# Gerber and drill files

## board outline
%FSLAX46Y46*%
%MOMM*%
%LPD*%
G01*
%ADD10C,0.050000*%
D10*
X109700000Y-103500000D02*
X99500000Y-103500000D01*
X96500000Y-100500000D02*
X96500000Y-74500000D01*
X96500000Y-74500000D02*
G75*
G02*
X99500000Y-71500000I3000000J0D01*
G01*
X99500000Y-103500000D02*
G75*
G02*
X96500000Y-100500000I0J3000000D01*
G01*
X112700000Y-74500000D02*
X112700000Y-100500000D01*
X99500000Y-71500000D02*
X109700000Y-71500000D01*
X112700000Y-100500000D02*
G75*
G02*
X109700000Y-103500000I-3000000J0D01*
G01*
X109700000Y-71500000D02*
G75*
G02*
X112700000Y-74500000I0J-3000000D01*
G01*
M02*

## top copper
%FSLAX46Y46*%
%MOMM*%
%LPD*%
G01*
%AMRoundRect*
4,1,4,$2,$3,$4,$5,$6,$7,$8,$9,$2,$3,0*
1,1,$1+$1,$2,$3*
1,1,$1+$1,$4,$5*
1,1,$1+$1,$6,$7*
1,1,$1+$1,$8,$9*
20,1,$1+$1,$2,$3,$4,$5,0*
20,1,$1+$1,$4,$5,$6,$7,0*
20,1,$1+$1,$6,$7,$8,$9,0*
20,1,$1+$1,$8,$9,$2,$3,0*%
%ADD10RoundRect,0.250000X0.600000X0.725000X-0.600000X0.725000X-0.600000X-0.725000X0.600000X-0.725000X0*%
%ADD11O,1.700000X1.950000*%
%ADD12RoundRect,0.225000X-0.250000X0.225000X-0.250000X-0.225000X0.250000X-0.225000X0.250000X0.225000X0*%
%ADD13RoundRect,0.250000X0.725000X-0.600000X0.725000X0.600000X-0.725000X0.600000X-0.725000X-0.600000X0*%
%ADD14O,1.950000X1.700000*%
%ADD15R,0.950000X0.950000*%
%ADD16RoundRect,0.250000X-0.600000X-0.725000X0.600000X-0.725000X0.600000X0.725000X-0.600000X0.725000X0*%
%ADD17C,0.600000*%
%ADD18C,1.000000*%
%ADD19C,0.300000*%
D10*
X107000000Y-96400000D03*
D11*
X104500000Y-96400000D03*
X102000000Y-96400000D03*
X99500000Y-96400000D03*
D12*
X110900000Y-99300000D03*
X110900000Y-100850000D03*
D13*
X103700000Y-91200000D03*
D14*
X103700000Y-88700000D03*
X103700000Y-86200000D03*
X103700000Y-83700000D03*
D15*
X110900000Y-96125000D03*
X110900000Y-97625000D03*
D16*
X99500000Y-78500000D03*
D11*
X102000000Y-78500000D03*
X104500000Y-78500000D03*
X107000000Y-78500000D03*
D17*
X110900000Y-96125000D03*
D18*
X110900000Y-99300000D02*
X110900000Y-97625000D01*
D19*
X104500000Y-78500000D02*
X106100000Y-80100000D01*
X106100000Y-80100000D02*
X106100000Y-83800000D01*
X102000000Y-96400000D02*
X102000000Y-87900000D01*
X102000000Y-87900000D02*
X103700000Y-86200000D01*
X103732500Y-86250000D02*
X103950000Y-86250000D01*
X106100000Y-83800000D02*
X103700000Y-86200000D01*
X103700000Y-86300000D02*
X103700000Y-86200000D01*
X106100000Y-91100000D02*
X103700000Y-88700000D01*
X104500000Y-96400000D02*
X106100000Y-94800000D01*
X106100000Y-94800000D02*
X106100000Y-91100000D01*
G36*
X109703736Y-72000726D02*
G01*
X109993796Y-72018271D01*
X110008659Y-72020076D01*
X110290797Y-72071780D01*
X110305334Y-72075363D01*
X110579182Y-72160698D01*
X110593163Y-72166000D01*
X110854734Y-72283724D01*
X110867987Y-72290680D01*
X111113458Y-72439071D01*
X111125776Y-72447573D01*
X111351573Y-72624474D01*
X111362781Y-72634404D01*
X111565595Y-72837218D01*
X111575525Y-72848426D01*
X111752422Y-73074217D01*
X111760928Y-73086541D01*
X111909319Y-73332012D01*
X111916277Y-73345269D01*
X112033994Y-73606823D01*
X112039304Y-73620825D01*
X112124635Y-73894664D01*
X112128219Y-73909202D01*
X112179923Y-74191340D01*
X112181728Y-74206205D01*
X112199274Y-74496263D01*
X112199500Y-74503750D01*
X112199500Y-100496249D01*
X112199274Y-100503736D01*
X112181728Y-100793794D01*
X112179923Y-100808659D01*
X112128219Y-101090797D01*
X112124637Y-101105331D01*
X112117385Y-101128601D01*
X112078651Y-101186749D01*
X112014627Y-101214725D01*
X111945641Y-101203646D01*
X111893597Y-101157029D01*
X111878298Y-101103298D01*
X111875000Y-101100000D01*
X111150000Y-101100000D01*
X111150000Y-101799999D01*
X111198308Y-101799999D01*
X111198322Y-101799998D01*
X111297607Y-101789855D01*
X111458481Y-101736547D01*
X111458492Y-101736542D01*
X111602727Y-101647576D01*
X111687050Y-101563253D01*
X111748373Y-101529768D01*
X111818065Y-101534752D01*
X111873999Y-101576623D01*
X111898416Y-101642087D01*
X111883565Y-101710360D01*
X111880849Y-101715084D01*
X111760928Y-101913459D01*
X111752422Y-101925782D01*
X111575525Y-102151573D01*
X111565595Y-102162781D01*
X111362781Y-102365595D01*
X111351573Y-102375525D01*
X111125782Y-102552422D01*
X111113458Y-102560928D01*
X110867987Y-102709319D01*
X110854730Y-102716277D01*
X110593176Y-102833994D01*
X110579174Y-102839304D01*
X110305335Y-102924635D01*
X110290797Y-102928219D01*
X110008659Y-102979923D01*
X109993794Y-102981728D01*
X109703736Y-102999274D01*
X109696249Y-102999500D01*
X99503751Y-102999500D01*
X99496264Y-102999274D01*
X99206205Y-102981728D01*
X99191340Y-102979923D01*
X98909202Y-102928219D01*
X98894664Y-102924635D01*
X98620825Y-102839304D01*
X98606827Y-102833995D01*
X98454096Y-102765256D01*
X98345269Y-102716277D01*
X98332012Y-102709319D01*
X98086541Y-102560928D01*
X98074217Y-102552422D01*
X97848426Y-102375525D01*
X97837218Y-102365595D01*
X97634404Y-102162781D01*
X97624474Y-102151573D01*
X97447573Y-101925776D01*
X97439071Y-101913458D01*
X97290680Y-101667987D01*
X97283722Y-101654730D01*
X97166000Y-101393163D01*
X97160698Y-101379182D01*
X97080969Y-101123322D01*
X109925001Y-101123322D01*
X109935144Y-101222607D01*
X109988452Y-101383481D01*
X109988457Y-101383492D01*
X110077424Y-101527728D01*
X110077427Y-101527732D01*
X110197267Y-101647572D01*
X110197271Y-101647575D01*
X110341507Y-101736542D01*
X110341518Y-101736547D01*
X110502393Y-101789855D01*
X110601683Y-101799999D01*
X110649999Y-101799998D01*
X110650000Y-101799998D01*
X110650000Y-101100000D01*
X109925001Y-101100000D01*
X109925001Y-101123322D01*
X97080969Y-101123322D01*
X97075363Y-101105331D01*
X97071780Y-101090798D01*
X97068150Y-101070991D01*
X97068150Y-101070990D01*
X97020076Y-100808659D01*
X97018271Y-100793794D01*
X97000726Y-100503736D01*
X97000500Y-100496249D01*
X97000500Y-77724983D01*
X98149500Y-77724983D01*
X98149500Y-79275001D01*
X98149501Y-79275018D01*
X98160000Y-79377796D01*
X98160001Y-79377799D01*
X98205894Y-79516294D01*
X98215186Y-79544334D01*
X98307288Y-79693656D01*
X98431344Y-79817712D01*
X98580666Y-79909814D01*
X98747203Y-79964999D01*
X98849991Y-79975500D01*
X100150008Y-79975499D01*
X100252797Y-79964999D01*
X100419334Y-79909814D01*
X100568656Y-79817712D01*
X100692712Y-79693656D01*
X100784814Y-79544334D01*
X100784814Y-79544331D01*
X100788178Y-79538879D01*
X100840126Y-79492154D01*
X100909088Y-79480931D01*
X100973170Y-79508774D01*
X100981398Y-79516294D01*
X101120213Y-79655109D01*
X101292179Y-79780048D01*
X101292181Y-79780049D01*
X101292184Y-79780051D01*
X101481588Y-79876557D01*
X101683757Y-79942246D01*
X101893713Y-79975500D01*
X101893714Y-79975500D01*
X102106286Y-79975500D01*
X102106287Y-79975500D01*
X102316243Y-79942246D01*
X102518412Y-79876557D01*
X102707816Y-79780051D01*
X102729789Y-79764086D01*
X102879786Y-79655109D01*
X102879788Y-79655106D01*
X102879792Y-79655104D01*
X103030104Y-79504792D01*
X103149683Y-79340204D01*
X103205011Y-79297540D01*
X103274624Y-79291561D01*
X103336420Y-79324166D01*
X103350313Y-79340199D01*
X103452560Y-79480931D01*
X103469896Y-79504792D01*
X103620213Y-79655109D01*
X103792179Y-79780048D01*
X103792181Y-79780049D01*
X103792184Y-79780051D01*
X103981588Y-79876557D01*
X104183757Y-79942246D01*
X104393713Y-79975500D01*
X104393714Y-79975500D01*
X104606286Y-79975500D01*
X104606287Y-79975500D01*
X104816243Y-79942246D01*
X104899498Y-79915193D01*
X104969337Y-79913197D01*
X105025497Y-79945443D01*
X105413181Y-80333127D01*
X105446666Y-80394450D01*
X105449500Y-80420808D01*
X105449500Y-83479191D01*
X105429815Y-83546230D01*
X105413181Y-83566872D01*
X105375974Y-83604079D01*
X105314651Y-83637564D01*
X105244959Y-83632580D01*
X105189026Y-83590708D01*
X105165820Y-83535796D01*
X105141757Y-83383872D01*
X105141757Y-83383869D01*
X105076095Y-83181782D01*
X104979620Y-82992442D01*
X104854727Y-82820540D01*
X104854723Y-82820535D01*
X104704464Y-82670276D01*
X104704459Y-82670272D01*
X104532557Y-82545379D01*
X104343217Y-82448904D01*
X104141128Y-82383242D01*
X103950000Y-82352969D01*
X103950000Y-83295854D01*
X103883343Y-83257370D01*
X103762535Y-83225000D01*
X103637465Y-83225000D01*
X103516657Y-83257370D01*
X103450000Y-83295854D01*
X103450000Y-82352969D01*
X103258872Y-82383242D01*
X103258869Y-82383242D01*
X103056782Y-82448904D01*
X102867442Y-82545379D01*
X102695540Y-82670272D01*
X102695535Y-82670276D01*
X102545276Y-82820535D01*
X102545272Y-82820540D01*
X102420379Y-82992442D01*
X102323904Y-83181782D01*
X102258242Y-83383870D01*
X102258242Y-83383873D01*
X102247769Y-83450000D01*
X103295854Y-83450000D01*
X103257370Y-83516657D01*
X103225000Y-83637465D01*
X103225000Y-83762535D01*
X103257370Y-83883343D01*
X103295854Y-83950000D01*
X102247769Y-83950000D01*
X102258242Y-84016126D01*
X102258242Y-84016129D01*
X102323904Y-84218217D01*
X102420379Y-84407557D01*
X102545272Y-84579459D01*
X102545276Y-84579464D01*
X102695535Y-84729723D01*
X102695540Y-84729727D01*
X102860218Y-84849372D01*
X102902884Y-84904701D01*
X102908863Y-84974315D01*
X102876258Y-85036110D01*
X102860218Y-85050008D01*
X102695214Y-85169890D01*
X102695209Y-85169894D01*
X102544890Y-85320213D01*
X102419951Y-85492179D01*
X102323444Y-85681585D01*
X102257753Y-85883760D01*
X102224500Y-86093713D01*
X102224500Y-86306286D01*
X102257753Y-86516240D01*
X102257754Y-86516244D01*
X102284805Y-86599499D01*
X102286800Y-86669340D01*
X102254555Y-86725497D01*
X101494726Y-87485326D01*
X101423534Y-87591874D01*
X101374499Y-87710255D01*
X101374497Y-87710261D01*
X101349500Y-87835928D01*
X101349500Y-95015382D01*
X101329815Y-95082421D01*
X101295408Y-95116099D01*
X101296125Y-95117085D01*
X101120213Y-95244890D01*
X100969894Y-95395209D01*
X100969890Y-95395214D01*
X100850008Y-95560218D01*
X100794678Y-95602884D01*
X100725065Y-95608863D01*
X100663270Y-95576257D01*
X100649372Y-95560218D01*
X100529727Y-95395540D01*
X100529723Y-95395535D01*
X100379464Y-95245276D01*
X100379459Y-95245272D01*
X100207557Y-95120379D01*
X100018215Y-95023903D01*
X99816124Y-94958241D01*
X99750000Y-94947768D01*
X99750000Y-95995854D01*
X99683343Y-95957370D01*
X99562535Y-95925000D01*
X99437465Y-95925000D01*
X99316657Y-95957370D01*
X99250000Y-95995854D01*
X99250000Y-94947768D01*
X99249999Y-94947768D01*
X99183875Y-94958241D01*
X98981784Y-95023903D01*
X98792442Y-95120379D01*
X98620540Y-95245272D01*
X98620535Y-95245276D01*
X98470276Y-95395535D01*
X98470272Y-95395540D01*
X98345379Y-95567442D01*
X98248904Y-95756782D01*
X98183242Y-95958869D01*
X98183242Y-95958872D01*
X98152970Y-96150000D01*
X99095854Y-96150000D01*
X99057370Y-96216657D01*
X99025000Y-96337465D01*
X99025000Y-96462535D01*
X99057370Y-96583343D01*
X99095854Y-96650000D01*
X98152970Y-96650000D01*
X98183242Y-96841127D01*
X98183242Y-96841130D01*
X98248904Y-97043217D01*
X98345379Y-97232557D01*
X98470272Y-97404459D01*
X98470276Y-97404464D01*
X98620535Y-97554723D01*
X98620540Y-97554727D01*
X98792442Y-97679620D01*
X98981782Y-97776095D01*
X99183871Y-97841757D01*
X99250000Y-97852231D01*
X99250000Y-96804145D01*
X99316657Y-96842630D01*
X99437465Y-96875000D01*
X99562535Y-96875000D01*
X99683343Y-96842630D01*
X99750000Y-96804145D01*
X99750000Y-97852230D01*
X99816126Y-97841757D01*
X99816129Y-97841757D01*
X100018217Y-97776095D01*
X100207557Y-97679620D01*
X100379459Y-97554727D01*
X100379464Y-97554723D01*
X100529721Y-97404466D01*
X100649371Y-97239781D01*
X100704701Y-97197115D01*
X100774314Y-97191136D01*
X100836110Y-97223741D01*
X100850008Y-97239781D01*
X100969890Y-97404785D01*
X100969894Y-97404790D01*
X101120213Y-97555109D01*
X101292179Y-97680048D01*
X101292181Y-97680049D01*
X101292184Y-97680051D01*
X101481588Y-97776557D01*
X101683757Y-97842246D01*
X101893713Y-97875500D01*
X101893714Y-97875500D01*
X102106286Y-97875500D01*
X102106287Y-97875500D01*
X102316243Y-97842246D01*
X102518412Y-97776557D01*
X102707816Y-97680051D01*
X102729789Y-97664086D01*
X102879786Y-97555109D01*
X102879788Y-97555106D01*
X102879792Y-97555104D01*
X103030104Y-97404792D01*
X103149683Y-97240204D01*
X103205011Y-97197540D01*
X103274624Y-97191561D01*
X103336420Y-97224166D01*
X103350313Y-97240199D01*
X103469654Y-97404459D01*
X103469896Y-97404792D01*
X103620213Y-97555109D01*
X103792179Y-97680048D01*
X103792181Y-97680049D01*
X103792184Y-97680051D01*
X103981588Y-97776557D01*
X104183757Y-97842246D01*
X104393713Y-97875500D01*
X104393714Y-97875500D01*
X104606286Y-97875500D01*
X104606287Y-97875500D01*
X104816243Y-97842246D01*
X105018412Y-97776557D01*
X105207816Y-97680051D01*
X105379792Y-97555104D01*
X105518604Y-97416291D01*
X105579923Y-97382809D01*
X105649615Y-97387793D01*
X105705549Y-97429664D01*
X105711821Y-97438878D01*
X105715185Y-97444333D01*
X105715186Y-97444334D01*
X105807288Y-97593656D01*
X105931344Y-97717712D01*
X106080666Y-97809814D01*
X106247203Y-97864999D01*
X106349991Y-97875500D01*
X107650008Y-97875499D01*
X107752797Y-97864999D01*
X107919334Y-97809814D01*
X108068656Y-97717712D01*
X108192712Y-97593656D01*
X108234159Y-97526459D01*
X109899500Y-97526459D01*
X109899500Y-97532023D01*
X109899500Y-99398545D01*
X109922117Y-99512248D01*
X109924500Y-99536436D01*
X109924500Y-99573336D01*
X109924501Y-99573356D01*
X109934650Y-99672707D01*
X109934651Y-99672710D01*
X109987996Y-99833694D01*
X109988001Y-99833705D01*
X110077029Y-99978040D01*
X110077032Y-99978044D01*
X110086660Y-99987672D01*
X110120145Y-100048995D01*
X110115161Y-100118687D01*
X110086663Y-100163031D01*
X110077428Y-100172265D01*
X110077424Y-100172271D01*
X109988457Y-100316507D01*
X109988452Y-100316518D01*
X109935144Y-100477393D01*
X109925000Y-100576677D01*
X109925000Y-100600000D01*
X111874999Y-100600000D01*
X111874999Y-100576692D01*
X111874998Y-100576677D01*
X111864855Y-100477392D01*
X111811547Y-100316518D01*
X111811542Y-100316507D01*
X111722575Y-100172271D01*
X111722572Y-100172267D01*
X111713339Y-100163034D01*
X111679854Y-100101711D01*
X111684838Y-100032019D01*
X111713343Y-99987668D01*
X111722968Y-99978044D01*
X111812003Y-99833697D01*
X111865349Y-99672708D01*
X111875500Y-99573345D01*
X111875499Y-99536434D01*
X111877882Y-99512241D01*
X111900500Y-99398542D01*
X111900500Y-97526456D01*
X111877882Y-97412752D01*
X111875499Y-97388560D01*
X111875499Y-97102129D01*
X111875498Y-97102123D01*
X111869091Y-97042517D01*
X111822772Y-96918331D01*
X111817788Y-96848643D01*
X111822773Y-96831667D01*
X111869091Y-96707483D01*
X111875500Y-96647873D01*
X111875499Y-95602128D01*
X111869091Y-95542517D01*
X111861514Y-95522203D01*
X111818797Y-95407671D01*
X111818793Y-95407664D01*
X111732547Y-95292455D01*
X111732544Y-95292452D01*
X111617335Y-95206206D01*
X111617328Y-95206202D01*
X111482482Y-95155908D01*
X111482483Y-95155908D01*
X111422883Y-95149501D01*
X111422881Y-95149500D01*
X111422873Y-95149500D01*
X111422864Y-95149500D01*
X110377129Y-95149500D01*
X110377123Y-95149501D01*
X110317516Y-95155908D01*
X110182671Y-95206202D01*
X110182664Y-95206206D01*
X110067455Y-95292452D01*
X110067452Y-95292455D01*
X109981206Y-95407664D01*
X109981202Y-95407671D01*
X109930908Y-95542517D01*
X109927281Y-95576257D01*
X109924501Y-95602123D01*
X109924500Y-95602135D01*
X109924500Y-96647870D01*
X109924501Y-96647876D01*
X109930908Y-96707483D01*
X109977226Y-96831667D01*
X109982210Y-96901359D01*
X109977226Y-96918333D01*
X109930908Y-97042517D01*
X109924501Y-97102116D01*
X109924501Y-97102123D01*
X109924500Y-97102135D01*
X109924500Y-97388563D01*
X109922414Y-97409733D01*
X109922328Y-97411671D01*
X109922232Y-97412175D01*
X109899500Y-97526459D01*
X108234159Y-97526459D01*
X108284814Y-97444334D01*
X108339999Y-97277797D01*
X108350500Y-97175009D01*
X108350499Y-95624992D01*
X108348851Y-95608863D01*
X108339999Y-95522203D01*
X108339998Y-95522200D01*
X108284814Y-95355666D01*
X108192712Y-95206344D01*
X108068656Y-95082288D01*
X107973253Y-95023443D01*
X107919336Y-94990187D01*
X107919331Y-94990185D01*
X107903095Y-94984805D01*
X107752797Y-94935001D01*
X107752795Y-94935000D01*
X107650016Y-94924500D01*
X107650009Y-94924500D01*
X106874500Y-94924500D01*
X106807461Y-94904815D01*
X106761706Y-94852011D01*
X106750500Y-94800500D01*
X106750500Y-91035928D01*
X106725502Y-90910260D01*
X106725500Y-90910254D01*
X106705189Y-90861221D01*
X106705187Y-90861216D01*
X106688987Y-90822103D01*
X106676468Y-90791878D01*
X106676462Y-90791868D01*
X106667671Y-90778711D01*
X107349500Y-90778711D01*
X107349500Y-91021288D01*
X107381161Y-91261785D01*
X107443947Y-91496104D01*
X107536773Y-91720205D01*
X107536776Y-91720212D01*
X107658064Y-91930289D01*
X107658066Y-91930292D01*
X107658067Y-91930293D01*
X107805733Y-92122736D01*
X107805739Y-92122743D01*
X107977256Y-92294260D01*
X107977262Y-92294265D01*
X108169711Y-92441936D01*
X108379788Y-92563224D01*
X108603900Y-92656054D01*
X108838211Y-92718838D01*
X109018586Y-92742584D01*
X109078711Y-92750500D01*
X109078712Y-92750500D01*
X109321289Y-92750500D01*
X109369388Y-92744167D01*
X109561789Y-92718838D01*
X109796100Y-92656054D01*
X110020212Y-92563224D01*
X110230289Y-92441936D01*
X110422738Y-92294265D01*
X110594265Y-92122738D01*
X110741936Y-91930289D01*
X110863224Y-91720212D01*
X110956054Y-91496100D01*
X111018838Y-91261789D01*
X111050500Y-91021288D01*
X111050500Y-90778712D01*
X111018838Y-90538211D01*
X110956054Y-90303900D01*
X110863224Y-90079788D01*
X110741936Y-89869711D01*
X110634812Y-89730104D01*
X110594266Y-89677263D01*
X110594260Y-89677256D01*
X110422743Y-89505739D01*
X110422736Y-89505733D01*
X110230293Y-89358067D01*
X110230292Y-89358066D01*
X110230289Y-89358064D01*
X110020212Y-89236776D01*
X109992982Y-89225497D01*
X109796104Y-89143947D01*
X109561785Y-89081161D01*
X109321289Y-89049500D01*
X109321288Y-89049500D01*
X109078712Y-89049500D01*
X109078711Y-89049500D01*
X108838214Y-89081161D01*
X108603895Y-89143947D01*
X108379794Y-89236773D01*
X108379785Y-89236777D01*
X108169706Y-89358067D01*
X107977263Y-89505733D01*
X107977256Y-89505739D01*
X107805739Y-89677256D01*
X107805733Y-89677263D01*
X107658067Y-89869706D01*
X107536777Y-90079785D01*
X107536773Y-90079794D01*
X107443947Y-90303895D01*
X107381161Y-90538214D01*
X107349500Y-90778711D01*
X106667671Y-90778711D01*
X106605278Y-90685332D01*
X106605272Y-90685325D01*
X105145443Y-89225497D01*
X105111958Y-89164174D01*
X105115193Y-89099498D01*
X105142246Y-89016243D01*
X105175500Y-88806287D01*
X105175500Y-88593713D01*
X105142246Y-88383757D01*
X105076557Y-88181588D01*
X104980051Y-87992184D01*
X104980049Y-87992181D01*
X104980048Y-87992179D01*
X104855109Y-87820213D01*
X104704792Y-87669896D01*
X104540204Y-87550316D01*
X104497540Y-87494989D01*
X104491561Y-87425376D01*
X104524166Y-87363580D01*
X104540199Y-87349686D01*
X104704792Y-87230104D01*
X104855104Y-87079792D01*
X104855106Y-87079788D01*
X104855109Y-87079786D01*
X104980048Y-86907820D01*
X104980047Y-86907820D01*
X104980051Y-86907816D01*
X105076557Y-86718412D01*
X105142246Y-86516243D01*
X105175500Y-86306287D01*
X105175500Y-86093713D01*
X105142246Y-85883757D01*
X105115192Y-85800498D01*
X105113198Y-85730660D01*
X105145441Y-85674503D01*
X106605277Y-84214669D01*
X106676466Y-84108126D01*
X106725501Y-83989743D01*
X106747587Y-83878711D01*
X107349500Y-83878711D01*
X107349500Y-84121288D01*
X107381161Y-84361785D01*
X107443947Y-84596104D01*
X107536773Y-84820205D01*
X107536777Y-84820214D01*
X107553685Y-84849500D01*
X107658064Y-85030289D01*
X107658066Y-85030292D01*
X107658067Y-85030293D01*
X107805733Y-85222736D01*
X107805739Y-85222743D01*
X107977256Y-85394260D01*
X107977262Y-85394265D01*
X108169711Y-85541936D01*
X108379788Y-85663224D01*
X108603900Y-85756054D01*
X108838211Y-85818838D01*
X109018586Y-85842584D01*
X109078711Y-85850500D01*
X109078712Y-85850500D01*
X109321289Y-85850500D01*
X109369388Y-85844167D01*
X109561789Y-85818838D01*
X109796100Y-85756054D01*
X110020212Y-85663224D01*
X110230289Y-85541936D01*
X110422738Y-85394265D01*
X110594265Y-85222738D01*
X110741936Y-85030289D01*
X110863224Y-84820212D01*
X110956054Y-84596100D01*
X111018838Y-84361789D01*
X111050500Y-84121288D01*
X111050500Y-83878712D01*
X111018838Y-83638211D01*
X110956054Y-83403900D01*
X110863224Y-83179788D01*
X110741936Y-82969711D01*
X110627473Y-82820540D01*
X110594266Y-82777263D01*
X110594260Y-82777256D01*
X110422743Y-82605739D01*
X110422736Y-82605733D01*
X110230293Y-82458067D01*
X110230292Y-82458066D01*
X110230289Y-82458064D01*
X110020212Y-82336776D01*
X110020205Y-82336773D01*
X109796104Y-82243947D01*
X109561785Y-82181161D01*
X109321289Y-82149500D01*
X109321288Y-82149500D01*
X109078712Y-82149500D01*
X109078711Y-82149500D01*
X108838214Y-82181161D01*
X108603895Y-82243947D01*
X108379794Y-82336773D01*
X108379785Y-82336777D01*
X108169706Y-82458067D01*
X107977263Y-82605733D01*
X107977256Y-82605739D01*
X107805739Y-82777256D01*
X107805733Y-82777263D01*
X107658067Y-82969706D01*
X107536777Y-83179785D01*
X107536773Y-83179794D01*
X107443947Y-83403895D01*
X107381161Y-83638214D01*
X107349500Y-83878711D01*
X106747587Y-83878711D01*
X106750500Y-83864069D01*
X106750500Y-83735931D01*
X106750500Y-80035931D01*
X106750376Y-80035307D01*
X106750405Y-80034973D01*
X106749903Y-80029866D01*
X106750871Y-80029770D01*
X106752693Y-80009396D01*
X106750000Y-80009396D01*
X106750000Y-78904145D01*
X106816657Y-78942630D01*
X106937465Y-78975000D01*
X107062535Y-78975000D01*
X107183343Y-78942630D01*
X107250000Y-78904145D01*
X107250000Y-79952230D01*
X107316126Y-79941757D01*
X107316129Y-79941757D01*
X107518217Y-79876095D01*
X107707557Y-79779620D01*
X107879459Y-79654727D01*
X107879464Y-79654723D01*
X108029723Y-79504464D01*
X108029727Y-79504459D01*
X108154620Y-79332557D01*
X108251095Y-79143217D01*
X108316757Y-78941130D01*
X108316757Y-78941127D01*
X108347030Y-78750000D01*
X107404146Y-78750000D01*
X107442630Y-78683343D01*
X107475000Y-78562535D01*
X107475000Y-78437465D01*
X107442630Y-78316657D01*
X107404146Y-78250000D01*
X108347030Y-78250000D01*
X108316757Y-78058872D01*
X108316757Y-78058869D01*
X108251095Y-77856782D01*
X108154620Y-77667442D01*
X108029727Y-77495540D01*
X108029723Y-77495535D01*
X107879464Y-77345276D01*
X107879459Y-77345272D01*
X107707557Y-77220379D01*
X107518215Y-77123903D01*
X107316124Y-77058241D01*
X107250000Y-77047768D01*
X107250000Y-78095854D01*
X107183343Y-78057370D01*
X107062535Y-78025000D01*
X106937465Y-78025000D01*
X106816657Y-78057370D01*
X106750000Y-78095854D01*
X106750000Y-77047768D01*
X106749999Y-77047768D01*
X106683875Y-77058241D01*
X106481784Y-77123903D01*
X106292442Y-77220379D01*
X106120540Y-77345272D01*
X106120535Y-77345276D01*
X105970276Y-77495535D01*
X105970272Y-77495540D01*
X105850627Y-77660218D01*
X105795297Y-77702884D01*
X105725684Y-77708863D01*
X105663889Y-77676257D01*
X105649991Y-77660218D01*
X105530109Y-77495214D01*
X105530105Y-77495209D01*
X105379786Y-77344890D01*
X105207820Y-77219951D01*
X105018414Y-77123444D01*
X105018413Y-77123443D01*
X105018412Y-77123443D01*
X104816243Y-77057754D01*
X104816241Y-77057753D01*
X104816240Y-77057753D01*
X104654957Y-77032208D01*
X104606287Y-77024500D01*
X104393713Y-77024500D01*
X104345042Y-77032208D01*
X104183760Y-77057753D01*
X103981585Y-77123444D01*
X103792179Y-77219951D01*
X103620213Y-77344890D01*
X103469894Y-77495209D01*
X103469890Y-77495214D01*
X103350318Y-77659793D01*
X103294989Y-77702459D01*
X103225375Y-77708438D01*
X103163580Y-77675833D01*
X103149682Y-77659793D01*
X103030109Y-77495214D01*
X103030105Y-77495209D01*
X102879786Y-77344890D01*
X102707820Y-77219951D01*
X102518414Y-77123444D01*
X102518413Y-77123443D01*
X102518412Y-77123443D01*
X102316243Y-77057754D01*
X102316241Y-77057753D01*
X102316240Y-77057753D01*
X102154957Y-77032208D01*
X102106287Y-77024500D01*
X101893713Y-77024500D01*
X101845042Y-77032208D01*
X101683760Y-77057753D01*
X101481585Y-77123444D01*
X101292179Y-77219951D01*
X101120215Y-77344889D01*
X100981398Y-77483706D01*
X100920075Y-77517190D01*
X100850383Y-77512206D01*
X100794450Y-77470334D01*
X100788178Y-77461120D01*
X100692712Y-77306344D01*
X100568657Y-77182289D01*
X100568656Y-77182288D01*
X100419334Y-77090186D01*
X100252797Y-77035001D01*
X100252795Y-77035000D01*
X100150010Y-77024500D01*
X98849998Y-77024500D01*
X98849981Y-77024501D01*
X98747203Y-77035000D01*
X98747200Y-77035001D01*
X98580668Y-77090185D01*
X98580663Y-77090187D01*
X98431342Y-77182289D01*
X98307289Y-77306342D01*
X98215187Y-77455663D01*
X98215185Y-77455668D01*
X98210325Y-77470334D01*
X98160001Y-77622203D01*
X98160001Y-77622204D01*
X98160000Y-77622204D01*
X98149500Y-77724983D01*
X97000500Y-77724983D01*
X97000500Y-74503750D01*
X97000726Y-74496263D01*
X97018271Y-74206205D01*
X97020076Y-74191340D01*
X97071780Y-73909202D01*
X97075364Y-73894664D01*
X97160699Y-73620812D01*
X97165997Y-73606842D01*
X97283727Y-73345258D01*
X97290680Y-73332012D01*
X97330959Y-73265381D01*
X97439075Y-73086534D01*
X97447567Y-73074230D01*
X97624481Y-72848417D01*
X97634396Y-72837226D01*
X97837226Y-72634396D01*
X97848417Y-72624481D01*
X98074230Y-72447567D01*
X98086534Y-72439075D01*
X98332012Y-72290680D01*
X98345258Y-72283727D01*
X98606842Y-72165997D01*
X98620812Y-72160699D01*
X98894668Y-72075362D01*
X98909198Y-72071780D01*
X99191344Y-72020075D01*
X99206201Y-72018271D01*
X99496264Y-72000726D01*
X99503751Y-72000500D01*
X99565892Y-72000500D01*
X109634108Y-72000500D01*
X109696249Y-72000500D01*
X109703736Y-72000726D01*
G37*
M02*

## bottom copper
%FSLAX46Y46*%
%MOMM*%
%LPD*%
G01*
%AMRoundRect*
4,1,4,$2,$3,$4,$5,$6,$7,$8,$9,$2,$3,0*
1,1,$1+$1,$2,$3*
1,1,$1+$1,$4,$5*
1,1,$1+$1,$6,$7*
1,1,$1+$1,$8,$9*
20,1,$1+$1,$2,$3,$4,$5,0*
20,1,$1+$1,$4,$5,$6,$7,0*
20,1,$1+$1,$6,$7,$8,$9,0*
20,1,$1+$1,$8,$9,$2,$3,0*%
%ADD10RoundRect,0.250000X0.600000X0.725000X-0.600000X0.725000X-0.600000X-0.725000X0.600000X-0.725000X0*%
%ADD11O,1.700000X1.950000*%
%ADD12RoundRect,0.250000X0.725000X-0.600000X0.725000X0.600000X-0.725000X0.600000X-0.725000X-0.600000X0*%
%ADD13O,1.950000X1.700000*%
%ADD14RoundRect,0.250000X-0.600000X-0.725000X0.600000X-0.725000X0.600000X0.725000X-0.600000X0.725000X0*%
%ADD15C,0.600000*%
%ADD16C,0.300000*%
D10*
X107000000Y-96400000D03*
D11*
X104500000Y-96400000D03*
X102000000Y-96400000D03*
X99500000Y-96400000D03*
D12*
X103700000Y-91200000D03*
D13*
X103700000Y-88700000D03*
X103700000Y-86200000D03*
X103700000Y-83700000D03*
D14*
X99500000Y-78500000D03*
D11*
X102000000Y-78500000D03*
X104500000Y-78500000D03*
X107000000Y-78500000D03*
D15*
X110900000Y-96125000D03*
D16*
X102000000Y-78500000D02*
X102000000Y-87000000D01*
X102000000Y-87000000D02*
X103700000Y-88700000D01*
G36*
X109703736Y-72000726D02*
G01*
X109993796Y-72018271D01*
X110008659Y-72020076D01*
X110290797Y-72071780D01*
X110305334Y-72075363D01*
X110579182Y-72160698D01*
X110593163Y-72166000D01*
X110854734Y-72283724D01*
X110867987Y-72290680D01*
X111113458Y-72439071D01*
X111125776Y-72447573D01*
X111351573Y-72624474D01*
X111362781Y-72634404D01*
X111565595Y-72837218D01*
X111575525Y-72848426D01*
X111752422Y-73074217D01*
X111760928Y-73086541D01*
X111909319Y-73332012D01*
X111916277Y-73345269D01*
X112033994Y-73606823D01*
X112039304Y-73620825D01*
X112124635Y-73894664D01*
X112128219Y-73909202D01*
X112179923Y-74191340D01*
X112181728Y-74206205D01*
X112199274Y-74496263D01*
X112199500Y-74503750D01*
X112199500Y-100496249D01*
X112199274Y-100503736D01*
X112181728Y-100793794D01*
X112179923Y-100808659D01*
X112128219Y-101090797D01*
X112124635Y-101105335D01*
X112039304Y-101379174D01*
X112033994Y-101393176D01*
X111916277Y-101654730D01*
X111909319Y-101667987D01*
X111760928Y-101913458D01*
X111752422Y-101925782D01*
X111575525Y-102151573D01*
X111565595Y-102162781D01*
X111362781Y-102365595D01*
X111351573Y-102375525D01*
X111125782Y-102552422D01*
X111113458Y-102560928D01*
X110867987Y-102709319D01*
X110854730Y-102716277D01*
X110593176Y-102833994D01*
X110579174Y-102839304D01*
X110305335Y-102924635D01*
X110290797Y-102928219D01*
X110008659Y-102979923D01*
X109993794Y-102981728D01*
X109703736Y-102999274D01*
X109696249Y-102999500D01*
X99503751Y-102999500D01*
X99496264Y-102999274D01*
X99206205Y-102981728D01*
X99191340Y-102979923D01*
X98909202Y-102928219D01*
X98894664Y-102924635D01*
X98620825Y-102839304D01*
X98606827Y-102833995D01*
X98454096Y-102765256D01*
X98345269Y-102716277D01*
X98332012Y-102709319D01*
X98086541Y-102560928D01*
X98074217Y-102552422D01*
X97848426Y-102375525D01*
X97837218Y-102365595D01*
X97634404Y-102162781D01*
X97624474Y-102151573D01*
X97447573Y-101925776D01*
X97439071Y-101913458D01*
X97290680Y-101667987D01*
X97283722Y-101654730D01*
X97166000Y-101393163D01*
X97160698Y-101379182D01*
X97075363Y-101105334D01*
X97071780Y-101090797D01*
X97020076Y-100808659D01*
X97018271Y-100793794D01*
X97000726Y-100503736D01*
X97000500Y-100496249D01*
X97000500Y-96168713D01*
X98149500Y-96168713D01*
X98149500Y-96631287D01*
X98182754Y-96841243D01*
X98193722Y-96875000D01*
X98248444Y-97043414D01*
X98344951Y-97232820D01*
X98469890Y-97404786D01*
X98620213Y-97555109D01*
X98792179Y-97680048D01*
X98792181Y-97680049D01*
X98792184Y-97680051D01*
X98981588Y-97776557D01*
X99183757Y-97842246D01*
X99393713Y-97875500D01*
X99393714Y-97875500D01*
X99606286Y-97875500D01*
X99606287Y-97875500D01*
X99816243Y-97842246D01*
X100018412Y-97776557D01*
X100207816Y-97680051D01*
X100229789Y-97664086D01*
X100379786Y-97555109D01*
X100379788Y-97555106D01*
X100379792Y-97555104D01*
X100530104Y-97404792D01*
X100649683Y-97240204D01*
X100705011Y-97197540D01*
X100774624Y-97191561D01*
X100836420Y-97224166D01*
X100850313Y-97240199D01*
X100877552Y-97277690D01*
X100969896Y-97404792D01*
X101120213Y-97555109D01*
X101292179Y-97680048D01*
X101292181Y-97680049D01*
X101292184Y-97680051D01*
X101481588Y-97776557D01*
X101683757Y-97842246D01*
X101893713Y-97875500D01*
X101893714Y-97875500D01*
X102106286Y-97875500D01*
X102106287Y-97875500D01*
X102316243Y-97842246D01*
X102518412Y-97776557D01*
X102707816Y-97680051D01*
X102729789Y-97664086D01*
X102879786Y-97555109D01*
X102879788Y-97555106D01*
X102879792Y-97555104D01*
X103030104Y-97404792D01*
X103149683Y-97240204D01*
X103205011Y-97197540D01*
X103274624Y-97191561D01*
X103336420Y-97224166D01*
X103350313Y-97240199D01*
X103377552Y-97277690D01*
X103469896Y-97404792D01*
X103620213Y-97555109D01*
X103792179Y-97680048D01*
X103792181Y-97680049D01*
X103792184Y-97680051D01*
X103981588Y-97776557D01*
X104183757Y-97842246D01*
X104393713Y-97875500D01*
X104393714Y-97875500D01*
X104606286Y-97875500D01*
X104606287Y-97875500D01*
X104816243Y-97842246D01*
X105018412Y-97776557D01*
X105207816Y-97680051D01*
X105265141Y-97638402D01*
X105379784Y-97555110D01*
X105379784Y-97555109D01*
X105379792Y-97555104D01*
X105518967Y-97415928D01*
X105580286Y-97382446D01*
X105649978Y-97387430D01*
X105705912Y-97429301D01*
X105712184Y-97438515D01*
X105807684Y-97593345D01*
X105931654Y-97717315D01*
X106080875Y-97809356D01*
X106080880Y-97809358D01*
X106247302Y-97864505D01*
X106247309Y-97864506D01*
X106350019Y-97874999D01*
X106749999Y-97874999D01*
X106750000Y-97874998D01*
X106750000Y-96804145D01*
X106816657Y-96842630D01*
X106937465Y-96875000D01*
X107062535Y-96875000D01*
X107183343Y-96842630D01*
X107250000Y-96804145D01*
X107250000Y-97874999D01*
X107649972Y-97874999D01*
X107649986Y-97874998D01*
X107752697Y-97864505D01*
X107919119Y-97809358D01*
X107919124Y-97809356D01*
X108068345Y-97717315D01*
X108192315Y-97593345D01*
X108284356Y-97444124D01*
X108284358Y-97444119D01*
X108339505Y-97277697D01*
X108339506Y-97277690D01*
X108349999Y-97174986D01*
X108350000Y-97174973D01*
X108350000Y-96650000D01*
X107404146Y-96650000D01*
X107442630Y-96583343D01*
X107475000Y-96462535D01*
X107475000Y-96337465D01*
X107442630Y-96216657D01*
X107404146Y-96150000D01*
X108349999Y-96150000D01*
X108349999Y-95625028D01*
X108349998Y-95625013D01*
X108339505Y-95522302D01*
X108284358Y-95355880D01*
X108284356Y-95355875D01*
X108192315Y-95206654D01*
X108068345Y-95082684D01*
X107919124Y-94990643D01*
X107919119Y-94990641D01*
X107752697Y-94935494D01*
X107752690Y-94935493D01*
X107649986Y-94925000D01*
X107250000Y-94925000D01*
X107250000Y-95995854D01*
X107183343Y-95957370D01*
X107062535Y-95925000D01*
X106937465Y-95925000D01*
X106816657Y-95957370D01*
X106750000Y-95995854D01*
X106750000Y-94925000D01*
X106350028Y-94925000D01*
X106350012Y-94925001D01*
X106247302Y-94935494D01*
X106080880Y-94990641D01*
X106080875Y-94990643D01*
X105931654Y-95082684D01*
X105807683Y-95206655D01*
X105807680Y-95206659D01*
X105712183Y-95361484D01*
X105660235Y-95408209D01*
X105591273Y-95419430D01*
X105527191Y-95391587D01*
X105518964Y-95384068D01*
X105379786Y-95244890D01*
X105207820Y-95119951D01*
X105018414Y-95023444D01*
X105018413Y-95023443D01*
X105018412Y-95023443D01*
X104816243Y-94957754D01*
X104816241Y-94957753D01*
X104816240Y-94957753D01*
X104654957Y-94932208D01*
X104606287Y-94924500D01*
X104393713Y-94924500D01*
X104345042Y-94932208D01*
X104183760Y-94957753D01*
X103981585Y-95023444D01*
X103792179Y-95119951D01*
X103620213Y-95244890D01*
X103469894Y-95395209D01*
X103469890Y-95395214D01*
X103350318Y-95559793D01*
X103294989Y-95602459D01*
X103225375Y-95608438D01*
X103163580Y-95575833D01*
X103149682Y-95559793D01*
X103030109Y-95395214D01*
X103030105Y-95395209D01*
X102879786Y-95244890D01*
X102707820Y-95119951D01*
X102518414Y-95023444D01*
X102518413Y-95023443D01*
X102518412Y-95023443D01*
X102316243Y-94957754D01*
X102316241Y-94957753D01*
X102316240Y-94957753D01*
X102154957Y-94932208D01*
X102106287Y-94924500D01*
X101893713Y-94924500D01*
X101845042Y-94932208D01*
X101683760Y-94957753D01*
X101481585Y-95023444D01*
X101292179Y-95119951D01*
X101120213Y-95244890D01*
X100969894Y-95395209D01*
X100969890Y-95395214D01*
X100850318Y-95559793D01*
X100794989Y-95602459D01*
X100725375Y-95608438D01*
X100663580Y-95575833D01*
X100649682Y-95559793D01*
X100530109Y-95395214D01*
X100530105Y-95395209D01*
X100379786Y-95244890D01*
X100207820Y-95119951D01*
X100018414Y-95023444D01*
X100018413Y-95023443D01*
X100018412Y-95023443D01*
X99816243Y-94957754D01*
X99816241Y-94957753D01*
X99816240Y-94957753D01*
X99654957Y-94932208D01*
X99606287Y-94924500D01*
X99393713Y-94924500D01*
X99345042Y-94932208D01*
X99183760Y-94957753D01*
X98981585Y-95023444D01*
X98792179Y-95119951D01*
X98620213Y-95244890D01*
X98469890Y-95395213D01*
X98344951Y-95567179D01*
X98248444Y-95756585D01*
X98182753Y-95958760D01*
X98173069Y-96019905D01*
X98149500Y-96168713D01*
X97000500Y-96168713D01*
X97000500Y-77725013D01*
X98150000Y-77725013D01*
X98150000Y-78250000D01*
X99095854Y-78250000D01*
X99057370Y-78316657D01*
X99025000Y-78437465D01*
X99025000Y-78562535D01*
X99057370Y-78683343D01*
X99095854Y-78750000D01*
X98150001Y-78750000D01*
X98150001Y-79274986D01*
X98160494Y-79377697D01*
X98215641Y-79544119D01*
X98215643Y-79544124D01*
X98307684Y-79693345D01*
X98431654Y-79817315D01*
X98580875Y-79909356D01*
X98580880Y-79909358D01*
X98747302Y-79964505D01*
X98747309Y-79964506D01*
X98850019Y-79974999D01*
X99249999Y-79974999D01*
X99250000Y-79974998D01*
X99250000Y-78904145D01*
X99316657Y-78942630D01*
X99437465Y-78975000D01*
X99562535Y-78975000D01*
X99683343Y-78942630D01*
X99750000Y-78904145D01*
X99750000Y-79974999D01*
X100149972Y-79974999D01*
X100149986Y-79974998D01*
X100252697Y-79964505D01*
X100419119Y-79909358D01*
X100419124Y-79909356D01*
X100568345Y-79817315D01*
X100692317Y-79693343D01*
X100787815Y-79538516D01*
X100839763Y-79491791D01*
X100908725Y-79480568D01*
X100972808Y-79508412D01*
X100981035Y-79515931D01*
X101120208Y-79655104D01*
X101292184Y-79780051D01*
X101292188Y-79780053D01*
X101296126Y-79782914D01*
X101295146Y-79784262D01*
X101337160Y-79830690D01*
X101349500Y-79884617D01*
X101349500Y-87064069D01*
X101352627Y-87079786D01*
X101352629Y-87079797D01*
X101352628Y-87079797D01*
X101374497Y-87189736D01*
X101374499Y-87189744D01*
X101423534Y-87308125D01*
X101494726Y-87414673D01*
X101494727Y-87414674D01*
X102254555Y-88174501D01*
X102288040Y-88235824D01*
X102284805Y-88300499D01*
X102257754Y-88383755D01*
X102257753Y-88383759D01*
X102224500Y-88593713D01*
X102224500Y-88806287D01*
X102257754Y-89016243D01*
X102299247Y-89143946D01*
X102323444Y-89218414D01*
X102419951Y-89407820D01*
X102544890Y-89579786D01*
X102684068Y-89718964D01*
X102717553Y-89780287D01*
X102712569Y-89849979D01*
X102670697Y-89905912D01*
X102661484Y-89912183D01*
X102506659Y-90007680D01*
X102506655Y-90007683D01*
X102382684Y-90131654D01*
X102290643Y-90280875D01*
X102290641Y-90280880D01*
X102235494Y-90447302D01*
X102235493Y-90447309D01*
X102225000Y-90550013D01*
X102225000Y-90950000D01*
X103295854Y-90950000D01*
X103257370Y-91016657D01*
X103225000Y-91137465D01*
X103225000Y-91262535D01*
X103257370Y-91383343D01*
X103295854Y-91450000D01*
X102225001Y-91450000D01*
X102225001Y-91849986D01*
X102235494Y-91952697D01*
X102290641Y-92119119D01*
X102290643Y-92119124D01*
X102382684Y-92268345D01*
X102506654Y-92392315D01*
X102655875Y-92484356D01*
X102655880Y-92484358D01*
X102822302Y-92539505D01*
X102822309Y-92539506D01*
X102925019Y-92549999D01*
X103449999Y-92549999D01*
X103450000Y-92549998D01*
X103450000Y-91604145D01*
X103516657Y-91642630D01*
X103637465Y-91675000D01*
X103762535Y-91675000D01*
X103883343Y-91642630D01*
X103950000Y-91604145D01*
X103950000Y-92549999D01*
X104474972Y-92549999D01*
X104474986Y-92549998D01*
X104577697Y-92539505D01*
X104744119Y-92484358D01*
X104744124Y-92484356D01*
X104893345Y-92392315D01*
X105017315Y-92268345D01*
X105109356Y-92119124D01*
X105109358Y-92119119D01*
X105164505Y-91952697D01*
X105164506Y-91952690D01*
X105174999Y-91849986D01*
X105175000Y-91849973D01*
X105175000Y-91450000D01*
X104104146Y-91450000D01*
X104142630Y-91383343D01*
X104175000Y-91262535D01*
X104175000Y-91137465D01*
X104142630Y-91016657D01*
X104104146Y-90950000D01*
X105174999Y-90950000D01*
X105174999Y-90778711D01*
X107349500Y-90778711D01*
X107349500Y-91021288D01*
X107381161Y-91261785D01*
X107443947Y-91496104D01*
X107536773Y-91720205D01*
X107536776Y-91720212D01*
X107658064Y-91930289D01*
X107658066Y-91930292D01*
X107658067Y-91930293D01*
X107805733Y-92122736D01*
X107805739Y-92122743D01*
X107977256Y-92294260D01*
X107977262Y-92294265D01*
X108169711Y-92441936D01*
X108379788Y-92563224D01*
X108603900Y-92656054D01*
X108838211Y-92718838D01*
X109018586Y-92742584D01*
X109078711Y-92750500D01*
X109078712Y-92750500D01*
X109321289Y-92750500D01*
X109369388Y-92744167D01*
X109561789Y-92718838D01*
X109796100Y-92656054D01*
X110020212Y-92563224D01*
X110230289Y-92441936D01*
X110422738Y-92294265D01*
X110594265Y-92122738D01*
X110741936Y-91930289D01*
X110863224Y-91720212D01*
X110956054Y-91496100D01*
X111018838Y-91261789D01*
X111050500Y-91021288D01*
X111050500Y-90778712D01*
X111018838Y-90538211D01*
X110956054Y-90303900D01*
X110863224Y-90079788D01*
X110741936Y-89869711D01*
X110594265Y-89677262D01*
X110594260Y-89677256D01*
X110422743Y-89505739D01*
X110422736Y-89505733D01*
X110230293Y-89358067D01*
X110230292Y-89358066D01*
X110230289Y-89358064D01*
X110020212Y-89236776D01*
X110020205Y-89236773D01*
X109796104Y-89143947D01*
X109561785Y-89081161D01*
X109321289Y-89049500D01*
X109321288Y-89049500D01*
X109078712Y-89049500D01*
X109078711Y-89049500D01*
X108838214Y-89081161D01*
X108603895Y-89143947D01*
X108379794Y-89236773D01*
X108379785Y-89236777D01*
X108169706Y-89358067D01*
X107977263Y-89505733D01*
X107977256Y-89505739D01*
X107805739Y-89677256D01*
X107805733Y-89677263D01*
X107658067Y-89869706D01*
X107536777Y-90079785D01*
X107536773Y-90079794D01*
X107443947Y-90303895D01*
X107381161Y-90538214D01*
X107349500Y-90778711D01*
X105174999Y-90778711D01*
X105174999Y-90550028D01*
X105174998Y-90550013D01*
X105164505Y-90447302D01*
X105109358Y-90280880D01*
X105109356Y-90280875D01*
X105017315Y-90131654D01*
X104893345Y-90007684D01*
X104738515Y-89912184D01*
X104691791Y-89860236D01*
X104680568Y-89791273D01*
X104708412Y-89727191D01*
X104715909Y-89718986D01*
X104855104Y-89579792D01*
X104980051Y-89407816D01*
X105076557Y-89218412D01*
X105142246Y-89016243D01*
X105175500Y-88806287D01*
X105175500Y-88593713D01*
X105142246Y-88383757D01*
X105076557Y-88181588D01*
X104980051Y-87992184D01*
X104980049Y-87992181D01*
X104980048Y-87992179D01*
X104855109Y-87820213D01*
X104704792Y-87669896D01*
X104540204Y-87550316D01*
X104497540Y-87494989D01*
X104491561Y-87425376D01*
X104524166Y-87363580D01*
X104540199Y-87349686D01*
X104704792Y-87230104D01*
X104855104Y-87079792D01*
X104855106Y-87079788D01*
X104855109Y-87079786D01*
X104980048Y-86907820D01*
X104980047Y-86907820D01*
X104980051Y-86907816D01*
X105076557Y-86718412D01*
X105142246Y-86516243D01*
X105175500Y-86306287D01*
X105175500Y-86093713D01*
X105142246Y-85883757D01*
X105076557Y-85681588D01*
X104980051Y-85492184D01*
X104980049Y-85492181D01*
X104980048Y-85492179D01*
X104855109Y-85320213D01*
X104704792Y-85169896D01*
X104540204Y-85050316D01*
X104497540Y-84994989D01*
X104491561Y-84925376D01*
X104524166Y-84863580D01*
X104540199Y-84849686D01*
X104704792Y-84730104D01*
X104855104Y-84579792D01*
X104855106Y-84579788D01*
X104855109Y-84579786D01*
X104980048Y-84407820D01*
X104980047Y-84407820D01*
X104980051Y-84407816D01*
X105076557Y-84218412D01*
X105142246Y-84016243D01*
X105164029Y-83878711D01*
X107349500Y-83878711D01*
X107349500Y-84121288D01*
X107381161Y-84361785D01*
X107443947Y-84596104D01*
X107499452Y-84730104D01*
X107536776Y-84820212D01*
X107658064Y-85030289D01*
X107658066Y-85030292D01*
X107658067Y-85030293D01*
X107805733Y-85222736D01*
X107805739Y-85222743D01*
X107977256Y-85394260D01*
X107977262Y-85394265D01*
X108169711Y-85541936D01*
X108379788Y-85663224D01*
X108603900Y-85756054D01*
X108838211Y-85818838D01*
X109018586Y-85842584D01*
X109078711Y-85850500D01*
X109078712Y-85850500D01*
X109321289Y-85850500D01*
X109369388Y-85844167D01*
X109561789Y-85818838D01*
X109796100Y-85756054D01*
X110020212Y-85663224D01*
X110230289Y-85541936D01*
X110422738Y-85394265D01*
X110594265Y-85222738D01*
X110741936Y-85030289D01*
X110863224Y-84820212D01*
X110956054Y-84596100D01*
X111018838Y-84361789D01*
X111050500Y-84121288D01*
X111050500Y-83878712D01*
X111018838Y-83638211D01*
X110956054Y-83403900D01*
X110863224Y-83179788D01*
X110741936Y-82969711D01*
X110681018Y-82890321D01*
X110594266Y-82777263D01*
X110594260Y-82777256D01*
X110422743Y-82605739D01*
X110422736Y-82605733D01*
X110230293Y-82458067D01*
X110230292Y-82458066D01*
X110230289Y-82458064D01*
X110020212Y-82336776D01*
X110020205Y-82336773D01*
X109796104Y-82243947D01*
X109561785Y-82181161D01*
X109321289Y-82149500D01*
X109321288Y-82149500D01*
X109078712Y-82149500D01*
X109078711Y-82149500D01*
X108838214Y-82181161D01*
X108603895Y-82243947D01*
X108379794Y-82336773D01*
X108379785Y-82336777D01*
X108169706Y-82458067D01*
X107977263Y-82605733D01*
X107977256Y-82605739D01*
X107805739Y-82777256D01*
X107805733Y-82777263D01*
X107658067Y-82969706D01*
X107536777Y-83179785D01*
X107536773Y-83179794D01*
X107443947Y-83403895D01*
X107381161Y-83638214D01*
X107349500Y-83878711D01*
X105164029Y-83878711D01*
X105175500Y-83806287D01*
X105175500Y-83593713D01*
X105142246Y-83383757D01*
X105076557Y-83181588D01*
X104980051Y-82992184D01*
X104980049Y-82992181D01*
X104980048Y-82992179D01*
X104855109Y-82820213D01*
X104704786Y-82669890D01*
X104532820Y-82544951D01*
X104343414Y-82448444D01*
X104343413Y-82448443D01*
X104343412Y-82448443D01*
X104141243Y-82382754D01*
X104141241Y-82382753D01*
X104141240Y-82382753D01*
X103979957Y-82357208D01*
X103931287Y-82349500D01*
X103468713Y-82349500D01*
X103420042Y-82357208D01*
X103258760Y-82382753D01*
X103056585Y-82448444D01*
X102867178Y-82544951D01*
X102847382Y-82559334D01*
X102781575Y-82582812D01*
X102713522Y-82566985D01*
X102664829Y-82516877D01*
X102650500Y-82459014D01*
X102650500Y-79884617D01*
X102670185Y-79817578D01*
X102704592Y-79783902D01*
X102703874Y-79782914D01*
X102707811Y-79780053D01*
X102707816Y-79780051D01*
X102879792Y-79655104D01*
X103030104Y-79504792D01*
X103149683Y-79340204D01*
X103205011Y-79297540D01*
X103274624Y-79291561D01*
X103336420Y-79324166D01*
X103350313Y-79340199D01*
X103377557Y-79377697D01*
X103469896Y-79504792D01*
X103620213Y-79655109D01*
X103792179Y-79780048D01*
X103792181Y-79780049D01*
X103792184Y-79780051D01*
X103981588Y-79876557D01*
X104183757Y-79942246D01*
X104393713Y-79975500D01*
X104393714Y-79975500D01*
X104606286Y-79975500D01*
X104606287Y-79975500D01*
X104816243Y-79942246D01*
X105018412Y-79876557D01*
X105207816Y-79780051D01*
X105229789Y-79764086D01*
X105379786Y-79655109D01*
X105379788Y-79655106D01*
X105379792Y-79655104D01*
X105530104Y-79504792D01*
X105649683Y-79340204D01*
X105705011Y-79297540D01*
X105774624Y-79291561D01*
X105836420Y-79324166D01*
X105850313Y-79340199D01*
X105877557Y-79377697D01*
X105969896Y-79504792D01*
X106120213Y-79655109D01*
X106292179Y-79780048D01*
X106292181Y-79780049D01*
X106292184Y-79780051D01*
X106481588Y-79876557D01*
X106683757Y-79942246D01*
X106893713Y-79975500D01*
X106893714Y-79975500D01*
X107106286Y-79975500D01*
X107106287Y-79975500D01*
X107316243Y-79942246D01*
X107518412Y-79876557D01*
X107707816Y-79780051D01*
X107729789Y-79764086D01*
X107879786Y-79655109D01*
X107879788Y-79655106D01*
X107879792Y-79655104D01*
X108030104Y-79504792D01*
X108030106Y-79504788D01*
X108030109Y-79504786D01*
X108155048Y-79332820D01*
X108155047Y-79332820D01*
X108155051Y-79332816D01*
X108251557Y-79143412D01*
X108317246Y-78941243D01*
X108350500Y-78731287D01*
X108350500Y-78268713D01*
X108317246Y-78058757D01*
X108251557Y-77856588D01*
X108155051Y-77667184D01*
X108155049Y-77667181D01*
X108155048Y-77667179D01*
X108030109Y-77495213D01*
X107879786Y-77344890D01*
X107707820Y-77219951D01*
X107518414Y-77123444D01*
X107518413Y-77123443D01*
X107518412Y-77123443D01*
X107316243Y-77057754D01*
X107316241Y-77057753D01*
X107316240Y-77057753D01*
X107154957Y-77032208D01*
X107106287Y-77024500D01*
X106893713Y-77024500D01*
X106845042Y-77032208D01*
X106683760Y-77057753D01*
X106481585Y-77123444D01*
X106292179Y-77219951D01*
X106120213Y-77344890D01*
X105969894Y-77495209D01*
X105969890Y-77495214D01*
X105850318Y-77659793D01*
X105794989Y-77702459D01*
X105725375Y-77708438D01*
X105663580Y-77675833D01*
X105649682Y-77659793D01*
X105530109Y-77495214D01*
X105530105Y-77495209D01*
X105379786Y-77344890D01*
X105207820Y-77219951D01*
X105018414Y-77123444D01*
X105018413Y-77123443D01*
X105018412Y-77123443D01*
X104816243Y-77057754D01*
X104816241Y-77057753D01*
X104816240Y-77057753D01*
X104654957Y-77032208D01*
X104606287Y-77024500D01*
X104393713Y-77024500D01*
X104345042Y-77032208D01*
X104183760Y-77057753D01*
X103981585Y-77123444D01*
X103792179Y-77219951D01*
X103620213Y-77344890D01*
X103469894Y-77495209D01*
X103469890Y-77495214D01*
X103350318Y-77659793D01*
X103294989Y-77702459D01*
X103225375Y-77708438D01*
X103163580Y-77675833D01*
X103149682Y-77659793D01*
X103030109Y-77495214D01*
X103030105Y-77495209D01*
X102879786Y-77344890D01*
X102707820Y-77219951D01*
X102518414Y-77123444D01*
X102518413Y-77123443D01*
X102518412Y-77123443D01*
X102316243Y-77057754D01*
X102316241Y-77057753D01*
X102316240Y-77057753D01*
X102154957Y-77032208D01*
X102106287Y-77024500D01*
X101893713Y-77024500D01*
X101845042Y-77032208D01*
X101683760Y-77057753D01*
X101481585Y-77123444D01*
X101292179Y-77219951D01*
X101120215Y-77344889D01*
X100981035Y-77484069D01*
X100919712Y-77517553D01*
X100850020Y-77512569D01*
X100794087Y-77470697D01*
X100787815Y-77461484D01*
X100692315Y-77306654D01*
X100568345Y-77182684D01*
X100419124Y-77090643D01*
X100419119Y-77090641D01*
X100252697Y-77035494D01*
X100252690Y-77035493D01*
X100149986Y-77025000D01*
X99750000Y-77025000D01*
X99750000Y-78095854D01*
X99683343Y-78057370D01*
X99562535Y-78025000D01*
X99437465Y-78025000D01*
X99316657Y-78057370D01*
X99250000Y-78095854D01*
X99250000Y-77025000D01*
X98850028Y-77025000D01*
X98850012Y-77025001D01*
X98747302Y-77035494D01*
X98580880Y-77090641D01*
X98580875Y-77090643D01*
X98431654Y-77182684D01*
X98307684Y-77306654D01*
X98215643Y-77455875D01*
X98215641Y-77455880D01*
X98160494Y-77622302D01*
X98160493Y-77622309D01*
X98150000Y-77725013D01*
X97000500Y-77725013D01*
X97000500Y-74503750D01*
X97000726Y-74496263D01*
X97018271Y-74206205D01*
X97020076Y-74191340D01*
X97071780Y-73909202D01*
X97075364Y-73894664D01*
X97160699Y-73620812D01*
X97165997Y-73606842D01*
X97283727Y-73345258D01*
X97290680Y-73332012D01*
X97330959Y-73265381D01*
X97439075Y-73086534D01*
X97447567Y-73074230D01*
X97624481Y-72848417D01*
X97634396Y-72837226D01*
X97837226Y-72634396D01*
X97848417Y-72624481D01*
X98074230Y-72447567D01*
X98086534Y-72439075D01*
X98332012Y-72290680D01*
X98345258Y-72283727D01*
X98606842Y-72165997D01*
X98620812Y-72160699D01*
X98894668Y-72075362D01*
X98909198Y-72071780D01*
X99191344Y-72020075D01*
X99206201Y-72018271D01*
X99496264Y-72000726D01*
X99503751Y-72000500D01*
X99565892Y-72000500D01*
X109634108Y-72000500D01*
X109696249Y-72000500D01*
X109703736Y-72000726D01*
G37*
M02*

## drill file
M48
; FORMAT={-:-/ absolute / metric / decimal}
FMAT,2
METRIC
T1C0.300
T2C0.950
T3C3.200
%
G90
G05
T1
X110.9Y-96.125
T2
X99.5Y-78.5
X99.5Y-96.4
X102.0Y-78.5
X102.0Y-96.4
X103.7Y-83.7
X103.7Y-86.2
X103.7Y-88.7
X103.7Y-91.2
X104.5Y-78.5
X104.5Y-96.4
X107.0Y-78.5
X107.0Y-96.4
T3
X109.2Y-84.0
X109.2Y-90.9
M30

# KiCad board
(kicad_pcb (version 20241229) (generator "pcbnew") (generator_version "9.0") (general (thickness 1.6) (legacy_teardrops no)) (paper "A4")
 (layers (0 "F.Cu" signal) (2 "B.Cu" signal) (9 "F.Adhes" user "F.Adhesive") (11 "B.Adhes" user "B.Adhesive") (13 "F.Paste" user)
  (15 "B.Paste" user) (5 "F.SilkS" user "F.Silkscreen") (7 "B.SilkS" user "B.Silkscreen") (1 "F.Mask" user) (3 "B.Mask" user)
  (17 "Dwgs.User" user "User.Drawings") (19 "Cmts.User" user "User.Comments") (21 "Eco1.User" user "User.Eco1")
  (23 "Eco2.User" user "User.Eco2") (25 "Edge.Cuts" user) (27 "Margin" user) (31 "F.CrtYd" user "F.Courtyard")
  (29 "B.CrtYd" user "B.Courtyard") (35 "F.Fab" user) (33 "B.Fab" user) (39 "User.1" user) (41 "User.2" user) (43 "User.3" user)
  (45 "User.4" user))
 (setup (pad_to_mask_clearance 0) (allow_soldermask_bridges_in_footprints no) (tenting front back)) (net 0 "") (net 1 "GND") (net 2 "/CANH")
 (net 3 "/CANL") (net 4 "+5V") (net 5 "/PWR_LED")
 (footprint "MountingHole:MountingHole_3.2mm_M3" (layer "F.Cu") (at 109.2 90.9)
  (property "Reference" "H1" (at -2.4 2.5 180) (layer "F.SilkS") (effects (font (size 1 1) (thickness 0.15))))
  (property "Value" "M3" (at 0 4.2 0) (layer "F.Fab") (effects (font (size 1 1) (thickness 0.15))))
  (pad "" np_thru_hole circle (at 0 0) (size 3.2 3.2) (drill 3.2) (layers "*.Cu" "*.Mask")))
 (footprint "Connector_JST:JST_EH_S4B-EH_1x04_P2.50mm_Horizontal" (layer "F.Cu") (at 107 96.4 180)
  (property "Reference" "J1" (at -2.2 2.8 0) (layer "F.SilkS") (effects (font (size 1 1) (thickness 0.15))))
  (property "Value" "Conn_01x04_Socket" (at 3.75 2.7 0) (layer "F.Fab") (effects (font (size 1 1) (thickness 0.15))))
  (pad "1" thru_hole roundrect (at 0 0 180) (size 1.7 1.95) (drill 0.95) (layers "*.Cu" "*.Mask") (remove_unused_layers no)
   (roundrect_rratio 0.147059) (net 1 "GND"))
  (pad "2" thru_hole oval (at 2.5 0 180) (size 1.7 1.95) (drill 0.95) (layers "*.Cu" "*.Mask") (remove_unused_layers no) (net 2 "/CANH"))
  (pad "3" thru_hole oval (at 5 0 180) (size 1.7 1.95) (drill 0.95) (layers "*.Cu" "*.Mask") (remove_unused_layers no) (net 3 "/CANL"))
  (pad "4" thru_hole oval (at 7.5 0 180) (size 1.7 1.95) (drill 0.95) (layers "*.Cu" "*.Mask") (remove_unused_layers no) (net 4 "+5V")))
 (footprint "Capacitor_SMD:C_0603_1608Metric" (layer "F.Cu") (at 110.9 100.075 -90)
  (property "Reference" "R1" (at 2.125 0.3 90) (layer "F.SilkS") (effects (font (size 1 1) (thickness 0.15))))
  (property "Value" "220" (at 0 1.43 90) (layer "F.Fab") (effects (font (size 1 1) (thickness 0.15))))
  (pad "1" smd roundrect (at -0.775 0 270) (size 0.9 0.95) (layers "F.Cu" "F.Mask" "F.Paste") (roundrect_rratio 0.25) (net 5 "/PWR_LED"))
  (pad "2" smd roundrect (at 0.775 0 270) (size 0.9 0.95) (layers "F.Cu" "F.Mask" "F.Paste") (roundrect_rratio 0.25) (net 4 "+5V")))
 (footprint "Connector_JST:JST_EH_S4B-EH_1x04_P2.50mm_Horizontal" (layer "F.Cu") (at 103.7 91.2 90)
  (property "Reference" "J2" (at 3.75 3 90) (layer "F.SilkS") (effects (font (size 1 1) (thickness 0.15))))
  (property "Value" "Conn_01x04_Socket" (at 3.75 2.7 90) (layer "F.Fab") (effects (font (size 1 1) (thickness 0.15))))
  (pad "1" thru_hole roundrect (at 0 0 90) (size 1.7 1.95) (drill 0.95) (layers "*.Cu" "*.Mask") (remove_unused_layers no)
   (roundrect_rratio 0.147059) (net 1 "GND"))
  (pad "2" thru_hole oval (at 2.5 0 90) (size 1.7 1.95) (drill 0.95) (layers "*.Cu" "*.Mask") (remove_unused_layers no) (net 2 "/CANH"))
  (pad "3" thru_hole oval (at 5 0 90) (size 1.7 1.95) (drill 0.95) (layers "*.Cu" "*.Mask") (remove_unused_layers no) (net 3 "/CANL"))
  (pad "4" thru_hole oval (at 7.5 0 90) (size 1.7 1.95) (drill 0.95) (layers "*.Cu" "*.Mask") (remove_unused_layers no) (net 4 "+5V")))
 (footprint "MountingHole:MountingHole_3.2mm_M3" (layer "F.Cu") (at 109.2 84)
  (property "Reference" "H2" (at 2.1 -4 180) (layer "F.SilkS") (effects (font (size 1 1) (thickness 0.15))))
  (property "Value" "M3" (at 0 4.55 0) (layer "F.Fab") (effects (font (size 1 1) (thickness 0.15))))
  (pad "" np_thru_hole circle (at 0 0) (size 3.2 3.2) (drill 3.2) (layers "*.Cu" "*.Mask")))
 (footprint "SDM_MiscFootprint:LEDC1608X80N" (layer "F.Cu") (at 110.9 96.875 -90)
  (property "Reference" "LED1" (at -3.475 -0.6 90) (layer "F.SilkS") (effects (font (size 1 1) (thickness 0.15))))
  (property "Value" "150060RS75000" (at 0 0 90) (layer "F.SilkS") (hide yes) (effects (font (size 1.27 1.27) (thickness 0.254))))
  (pad "1" smd rect (at -0.75 0) (size 0.95 0.95) (layers "F.Cu" "F.Mask" "F.Paste") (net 1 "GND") (thermal_bridge_angle 45))
  (pad "2" smd rect (at 0.75 0) (size 0.95 0.95) (layers "F.Cu" "F.Mask" "F.Paste") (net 5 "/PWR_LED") (thermal_bridge_angle 45)))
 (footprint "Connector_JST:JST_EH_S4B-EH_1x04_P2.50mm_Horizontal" (layer "F.Cu") (at 99.5 78.5)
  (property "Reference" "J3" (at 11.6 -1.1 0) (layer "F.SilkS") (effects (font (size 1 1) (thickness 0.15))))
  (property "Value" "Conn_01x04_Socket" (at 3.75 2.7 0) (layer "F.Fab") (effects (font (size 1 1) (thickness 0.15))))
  (pad "1" thru_hole roundrect (at 0 0) (size 1.7 1.95) (drill 0.95) (layers "*.Cu" "*.Mask") (remove_unused_layers no)
   (roundrect_rratio 0.147059) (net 1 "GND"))
  (pad "2" thru_hole oval (at 2.5 0) (size 1.7 1.95) (drill 0.95) (layers "*.Cu" "*.Mask") (remove_unused_layers no) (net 2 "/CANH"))
  (pad "3" thru_hole oval (at 5 0) (size 1.7 1.95) (drill 0.95) (layers "*.Cu" "*.Mask") (remove_unused_layers no) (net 3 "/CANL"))
  (pad "4" thru_hole oval (at 7.5 0) (size 1.7 1.95) (drill 0.95) (layers "*.Cu" "*.Mask") (remove_unused_layers no) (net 4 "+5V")))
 (gr_line (start 109.7 103.5) (end 99.5 103.5) (stroke (width 0.05) (type default)) (layer "Edge.Cuts"))
 (gr_line (start 96.5 100.5) (end 96.5 74.5) (stroke (width 0.05) (type default)) (layer "Edge.Cuts"))
 (gr_arc (start 96.5 74.5) (mid 97.37868 72.37868) (end 99.5 71.5) (stroke (width 0.05) (type default)) (layer "Edge.Cuts"))
 (gr_arc (start 99.5 103.5) (mid 97.37868 102.62132) (end 96.5 100.5) (stroke (width 0.05) (type default)) (layer "Edge.Cuts"))
 (gr_line (start 112.7 74.5) (end 112.7 100.5) (stroke (width 0.05) (type default)) (layer "Edge.Cuts"))
 (gr_line (start 99.5 71.5) (end 109.7 71.5) (stroke (width 0.05) (type default)) (layer "Edge.Cuts"))
 (gr_arc (start 112.7 100.5) (mid 111.82132 102.62132) (end 109.7 103.5) (stroke (width 0.05) (type default)) (layer "Edge.Cuts"))
 (gr_arc (start 109.7 71.5) (mid 111.82132 72.37868) (end 112.7 74.5) (stroke (width 0.05) (type default)) (layer "Edge.Cuts"))
 (via (at 110.9 96.125) (size 0.6) (drill 0.3) (layers "F.Cu" "B.Cu") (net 1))
 (segment (start 110.9 99.3) (end 110.9 97.625) (width 1) (layer "F.Cu") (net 5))
 (segment (start 104.5 78.5) (end 106.1 80.1) (width 0.3) (layer "F.Cu") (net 3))
 (segment (start 106.1 80.1) (end 106.1 83.8) (width 0.3) (layer "F.Cu") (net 3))
 (segment (start 102 96.4) (end 102 87.9) (width 0.3) (layer "F.Cu") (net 3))
 (segment (start 102 87.9) (end 103.7 86.2) (width 0.3) (layer "F.Cu") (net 3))
 (segment (start 103.7325 86.25) (end 103.95 86.25) (width 0.3) (layer "F.Cu") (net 3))
 (segment (start 106.1 83.8) (end 103.7 86.2) (width 0.3) (layer "F.Cu") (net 3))
 (segment (start 103.7 86.3) (end 103.7 86.2) (width 0.3) (layer "F.Cu") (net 3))
 (segment (start 106.1 91.1) (end 103.7 88.7) (width 0.3) (layer "F.Cu") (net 2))
 (segment (start 104.5 96.4) (end 106.1 94.8) (width 0.3) (layer "F.Cu") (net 2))
 (segment (start 106.1 94.8) (end 106.1 91.1) (width 0.3) (layer "F.Cu") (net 2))
 (segment (start 102 78.5) (end 102 87) (width 0.3) (layer "B.Cu") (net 2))
 (segment (start 102 87) (end 103.7 88.7) (width 0.3) (layer "B.Cu") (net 2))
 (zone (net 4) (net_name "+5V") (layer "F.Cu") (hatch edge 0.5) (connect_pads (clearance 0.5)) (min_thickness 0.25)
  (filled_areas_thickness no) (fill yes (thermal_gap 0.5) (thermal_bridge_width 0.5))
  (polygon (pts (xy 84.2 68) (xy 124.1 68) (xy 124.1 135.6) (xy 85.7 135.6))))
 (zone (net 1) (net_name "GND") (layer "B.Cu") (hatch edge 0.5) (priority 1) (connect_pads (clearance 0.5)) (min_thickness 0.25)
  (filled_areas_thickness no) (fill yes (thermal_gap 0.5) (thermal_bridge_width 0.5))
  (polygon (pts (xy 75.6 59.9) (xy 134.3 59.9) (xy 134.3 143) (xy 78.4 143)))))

